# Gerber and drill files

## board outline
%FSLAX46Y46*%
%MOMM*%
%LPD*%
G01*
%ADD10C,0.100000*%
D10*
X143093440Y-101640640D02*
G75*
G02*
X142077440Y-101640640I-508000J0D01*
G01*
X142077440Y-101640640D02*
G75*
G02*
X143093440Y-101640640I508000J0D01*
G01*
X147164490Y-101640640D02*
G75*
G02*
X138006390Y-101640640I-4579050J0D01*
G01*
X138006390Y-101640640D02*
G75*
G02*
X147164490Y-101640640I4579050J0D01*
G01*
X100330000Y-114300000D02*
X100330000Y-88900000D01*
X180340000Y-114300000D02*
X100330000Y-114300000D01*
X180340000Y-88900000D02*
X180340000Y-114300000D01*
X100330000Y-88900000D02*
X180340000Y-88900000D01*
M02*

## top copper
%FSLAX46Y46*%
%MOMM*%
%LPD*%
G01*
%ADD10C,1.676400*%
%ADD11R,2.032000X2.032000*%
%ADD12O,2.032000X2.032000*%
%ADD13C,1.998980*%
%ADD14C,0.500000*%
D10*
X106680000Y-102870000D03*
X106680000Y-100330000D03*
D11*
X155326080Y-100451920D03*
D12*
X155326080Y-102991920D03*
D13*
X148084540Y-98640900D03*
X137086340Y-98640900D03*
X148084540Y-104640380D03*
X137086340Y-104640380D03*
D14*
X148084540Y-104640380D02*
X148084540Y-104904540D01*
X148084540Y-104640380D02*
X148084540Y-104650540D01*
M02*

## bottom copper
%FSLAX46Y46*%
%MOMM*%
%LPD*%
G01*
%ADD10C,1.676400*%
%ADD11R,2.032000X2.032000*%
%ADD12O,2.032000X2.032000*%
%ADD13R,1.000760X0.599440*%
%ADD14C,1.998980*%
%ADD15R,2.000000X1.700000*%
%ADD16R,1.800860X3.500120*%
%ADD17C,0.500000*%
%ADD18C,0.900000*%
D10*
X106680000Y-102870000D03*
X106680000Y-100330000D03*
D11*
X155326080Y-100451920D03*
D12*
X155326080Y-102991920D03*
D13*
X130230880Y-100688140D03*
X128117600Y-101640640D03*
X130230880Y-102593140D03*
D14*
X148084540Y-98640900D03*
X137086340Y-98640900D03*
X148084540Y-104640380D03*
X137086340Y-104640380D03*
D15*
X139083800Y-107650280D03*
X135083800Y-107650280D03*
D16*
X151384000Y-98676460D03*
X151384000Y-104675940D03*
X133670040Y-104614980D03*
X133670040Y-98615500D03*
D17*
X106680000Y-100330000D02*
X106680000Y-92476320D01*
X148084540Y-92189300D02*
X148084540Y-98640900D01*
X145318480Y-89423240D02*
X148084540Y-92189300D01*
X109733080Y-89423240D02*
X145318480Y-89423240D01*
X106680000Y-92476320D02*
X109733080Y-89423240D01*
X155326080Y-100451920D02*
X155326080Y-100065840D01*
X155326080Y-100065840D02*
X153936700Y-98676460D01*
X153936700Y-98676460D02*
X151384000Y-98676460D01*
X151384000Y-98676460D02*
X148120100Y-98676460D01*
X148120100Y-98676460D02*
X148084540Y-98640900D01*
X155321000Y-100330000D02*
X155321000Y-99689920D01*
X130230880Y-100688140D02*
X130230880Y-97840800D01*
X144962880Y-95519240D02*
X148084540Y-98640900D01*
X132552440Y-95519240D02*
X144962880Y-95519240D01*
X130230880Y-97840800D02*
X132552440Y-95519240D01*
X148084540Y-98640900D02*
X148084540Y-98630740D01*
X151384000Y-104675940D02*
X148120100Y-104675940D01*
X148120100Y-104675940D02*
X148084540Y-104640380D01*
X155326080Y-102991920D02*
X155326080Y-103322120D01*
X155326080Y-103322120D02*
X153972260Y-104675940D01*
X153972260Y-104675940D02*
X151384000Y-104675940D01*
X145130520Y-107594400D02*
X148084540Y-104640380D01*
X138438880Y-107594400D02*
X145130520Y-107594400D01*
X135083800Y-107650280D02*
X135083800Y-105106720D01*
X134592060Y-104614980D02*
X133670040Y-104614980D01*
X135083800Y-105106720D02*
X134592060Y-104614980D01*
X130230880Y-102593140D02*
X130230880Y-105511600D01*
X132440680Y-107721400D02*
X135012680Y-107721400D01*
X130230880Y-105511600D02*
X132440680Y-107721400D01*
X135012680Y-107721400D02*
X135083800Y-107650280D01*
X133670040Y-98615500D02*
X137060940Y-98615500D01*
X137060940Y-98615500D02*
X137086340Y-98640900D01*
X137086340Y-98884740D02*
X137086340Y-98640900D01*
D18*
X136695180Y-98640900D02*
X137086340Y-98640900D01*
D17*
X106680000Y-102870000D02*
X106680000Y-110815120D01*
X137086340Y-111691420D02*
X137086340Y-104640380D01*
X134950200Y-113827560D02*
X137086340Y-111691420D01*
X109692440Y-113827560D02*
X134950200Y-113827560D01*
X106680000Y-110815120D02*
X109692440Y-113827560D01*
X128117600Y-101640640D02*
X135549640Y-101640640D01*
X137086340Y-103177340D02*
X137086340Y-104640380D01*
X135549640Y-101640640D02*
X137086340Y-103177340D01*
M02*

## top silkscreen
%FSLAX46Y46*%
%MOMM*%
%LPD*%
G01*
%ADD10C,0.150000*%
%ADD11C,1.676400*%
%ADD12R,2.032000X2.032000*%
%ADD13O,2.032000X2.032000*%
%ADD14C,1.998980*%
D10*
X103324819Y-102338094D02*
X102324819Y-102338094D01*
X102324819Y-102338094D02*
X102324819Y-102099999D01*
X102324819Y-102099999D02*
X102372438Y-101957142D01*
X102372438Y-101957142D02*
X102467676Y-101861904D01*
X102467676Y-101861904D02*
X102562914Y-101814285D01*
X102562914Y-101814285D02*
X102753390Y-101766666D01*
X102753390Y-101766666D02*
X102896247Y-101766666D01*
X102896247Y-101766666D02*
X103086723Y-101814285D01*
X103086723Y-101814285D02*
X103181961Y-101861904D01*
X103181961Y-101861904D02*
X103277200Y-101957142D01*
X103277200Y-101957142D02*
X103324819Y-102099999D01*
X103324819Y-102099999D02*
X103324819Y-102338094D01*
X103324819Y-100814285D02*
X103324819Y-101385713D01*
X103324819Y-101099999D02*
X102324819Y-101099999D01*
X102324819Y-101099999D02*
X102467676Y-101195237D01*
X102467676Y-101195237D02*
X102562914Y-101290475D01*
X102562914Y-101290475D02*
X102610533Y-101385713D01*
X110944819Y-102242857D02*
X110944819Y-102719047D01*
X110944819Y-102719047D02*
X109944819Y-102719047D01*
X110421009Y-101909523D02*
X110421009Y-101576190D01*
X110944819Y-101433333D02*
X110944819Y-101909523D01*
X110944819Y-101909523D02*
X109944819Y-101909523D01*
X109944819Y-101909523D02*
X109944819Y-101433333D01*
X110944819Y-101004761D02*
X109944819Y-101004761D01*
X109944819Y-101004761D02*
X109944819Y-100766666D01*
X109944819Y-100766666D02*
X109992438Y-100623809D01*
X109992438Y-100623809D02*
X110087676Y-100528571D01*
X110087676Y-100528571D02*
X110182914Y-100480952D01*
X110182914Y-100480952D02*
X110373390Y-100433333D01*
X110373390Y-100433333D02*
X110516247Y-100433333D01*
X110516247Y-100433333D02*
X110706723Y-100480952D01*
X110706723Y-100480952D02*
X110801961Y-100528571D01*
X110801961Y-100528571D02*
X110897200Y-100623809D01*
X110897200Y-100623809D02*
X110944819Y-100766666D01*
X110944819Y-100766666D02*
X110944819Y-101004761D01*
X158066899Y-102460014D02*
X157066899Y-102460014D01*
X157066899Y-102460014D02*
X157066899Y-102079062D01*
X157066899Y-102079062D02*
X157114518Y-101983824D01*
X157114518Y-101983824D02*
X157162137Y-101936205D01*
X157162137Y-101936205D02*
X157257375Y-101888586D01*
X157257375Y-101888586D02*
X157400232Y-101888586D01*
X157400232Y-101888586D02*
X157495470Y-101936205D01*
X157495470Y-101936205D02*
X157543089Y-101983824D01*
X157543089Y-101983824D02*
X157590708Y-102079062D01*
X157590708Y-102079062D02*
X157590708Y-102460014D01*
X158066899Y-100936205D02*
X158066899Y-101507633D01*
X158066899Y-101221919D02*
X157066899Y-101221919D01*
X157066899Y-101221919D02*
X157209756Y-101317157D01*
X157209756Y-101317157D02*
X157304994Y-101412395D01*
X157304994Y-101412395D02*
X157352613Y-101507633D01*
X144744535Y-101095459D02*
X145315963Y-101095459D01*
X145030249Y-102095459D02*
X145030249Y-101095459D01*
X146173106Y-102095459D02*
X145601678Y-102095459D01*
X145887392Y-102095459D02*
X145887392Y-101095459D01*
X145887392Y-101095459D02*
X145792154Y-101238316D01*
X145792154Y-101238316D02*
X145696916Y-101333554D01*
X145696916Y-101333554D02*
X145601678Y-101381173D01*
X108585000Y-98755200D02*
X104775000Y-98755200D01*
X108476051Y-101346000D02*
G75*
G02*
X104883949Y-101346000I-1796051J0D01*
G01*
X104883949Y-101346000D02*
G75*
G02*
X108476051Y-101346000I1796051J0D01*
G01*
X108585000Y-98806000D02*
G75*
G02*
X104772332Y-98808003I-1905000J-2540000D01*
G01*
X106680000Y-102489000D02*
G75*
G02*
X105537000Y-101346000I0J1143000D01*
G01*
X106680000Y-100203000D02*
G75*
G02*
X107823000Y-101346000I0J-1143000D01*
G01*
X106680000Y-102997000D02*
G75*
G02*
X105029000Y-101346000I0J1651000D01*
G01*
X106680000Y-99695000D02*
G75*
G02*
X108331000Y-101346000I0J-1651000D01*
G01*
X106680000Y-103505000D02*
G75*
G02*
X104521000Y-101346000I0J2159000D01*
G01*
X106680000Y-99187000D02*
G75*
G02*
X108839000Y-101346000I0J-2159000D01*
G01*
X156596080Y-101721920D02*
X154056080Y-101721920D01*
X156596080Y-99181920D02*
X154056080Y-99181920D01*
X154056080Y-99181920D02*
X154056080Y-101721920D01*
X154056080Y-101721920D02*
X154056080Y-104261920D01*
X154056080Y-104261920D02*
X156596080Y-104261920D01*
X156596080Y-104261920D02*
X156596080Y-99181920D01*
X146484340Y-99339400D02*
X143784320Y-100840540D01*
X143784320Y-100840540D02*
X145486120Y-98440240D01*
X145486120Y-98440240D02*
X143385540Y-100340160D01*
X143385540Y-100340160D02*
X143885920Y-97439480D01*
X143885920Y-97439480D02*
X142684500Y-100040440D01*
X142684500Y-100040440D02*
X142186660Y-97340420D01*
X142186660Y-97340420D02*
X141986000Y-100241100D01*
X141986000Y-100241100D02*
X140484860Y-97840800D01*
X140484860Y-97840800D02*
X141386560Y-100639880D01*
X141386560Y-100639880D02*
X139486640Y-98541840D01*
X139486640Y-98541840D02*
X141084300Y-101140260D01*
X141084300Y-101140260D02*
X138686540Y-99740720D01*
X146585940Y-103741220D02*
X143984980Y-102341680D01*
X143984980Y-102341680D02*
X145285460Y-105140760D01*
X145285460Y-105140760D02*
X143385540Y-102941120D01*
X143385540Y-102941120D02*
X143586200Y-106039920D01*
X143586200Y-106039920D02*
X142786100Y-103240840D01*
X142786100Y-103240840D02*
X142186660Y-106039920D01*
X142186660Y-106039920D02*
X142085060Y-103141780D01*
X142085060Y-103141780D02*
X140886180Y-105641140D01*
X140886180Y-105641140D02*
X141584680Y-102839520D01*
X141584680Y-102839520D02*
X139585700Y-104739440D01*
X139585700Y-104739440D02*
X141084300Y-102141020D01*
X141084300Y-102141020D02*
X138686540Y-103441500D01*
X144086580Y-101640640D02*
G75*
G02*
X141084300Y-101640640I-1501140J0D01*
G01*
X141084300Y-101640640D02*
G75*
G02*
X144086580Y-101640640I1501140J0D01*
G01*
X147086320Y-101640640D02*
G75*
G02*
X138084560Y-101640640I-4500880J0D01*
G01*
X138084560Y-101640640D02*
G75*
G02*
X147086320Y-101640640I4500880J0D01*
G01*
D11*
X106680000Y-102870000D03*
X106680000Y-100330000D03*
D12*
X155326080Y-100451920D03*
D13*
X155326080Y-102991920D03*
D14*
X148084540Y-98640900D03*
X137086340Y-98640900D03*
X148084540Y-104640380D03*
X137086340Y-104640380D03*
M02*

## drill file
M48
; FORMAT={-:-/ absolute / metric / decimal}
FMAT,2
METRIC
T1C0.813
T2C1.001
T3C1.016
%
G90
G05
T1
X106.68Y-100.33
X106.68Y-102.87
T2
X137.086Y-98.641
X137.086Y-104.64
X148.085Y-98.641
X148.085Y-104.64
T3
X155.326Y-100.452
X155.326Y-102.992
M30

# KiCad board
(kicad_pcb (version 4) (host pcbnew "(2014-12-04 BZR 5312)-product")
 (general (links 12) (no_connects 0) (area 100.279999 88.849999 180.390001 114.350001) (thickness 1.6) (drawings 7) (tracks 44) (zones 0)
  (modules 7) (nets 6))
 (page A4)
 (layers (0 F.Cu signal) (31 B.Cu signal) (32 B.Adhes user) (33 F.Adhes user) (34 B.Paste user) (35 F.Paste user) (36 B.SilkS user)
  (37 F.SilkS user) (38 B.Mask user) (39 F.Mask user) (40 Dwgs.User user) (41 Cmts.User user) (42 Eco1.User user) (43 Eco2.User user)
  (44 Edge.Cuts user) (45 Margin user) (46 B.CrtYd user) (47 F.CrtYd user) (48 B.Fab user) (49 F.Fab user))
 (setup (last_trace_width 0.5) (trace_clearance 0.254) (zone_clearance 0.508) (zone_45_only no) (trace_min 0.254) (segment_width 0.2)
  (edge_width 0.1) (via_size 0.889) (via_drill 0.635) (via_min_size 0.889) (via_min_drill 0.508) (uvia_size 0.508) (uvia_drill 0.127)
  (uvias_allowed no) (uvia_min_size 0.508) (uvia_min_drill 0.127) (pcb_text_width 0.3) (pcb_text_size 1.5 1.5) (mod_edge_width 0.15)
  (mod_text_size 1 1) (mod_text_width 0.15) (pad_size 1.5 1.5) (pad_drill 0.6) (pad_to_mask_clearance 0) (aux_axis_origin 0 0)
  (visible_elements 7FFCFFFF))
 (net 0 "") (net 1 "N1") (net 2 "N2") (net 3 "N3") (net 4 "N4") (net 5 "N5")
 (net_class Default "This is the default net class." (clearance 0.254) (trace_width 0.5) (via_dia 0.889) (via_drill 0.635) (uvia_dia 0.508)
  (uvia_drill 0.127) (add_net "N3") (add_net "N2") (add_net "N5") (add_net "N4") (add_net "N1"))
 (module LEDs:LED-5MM (layer F.Cu) (at 106.68 101.6 90)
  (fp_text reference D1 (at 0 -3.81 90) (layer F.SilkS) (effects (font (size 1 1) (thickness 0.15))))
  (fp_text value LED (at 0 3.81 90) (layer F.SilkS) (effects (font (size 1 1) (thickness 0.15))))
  (fp_line (start 2.8448 1.905) (end 2.8448 -1.905) (layer F.SilkS) (width 0.15))
  (fp_circle (center 0.254 0) (end -1.016 1.27) (layer F.SilkS) (width 0.15))
  (fp_arc (start 0.254 0) (end 2.794 1.905) (angle 286.2) (layer F.SilkS) (width 0.15))
  (fp_arc (start 0.254 0) (end -0.889 0) (angle 90) (layer F.SilkS) (width 0.15))
  (fp_arc (start 0.254 0) (end 1.397 0) (angle 90) (layer F.SilkS) (width 0.15))
  (fp_arc (start 0.254 0) (end -1.397 0) (angle 90) (layer F.SilkS) (width 0.15))
  (fp_arc (start 0.254 0) (end 1.905 0) (angle 90) (layer F.SilkS) (width 0.15))
  (fp_arc (start 0.254 0) (end -1.905 0) (angle 90) (layer F.SilkS) (width 0.15))
  (fp_arc (start 0.254 0) (end 2.413 0) (angle 90) (layer F.SilkS) (width 0.15))
  (pad 1 thru_hole circle (at -1.27 0 90) (size 1.6764 1.6764) (drill 0.8128) (layers *.Cu *.Mask F.SilkS) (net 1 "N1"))
  (pad 2 thru_hole circle (at 1.27 0 90) (size 1.6764 1.6764) (drill 0.8128) (layers *.Cu *.Mask F.SilkS) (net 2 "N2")))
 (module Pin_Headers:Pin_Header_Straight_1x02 (layer F.Cu) (at 155.32608 101.72192 270)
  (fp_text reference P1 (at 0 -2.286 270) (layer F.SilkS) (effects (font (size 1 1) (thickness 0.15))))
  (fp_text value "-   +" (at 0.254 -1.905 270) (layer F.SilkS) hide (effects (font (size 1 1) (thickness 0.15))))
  (fp_line (start 0 -1.27) (end 0 1.27) (layer F.SilkS) (width 0.15))
  (fp_line (start -2.54 -1.27) (end -2.54 1.27) (layer F.SilkS) (width 0.15))
  (fp_line (start -2.54 1.27) (end 0 1.27) (layer F.SilkS) (width 0.15))
  (fp_line (start 0 1.27) (end 2.54 1.27) (layer F.SilkS) (width 0.15))
  (fp_line (start 2.54 1.27) (end 2.54 -1.27) (layer F.SilkS) (width 0.15))
  (fp_line (start 2.54 -1.27) (end -2.54 -1.27) (layer F.SilkS) (width 0.15))
  (pad 1 thru_hole rect (at -1.27 0 270) (size 2.032 2.032) (drill 1.016) (layers *.Cu *.Mask F.SilkS) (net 2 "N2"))
  (pad 2 thru_hole oval (at 1.27 0 270) (size 2.032 2.032) (drill 1.016) (layers *.Cu *.Mask F.SilkS) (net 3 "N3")))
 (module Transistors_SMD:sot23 (layer B.Cu) (at 129.17424 101.64064 270)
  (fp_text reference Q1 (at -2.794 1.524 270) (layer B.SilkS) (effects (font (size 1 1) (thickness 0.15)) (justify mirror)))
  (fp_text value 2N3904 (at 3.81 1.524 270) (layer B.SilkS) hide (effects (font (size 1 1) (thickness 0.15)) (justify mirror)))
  (pad 1 smd rect (at -0.9525 -1.05664 270) (size 0.59944 1.00076) (layers B.Cu B.Paste B.Mask) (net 2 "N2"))
  (pad 3 smd rect (at 0 1.05664 270) (size 0.59944 1.00076) (layers B.Cu B.Paste B.Mask) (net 1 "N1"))
  (pad 2 smd rect (at 0.9525 -1.05664 270) (size 0.59944 1.00076) (layers B.Cu B.Paste B.Mask) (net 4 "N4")))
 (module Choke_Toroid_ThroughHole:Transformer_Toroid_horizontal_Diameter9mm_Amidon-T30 (layer F.Cu) (at 142.58544 101.64064 180)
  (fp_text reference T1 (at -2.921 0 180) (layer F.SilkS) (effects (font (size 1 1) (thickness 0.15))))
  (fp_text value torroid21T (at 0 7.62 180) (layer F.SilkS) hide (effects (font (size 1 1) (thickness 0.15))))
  (fp_line (start -3.8989 2.30124) (end -1.19888 0.8001) (layer F.SilkS) (width 0.15))
  (fp_line (start -1.19888 0.8001) (end -2.90068 3.2004) (layer F.SilkS) (width 0.15))
  (fp_line (start -2.90068 3.2004) (end -0.8001 1.30048) (layer F.SilkS) (width 0.15))
  (fp_line (start -0.8001 1.30048) (end -1.30048 4.20116) (layer F.SilkS) (width 0.15))
  (fp_line (start -1.30048 4.20116) (end -0.09906 1.6002) (layer F.SilkS) (width 0.15))
  (fp_line (start -0.09906 1.6002) (end 0.39878 4.30022) (layer F.SilkS) (width 0.15))
  (fp_line (start 0.39878 4.30022) (end 0.59944 1.39954) (layer F.SilkS) (width 0.15))
  (fp_line (start 0.59944 1.39954) (end 2.10058 3.79984) (layer F.SilkS) (width 0.15))
  (fp_line (start 2.10058 3.79984) (end 1.19888 1.00076) (layer F.SilkS) (width 0.15))
  (fp_line (start 1.19888 1.00076) (end 3.0988 3.0988) (layer F.SilkS) (width 0.15))
  (fp_line (start 3.0988 3.0988) (end 1.50114 0.50038) (layer F.SilkS) (width 0.15))
  (fp_line (start 1.50114 0.50038) (end 3.8989 1.89992) (layer F.SilkS) (width 0.15))
  (fp_line (start -4.0005 -2.10058) (end -1.39954 -0.70104) (layer F.SilkS) (width 0.15))
  (fp_line (start -1.39954 -0.70104) (end -2.70002 -3.50012) (layer F.SilkS) (width 0.15))
  (fp_line (start -2.70002 -3.50012) (end -0.8001 -1.30048) (layer F.SilkS) (width 0.15))
  (fp_line (start -0.8001 -1.30048) (end -1.00076 -4.39928) (layer F.SilkS) (width 0.15))
  (fp_line (start -1.00076 -4.39928) (end -0.20066 -1.6002) (layer F.SilkS) (width 0.15))
  (fp_line (start -0.20066 -1.6002) (end 0.39878 -4.39928) (layer F.SilkS) (width 0.15))
  (fp_line (start 0.39878 -4.39928) (end 0.50038 -1.50114) (layer F.SilkS) (width 0.15))
  (fp_line (start 0.50038 -1.50114) (end 1.69926 -4.0005) (layer F.SilkS) (width 0.15))
  (fp_line (start 1.69926 -4.0005) (end 1.00076 -1.19888) (layer F.SilkS) (width 0.15))
  (fp_line (start 1.00076 -1.19888) (end 2.99974 -3.0988) (layer F.SilkS) (width 0.15))
  (fp_line (start 2.99974 -3.0988) (end 1.50114 -0.50038) (layer F.SilkS) (width 0.15))
  (fp_line (start 1.50114 -0.50038) (end 3.8989 -1.80086) (layer F.SilkS) (width 0.15))
  (fp_circle (center 0 0) (end 1.50114 0) (layer F.SilkS) (width 0.15))
  (fp_circle (center 0 0) (end 4.50088 0) (layer F.SilkS) (width 0.15))
  (pad 1 thru_hole circle (at -5.4991 2.99974 180) (size 1.99898 1.99898) (drill 1.00076) (layers *.Cu *.Mask F.SilkS) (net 2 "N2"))
  (pad 2 thru_hole circle (at 5.4991 2.99974 180) (size 1.99898 1.99898) (drill 1.00076) (layers *.Cu *.Mask F.SilkS) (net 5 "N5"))
  (pad 3 thru_hole circle (at -5.4991 -2.99974 180) (size 1.99898 1.99898) (drill 1.00076) (layers *.Cu *.Mask F.SilkS) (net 3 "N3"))
  (pad 4 thru_hole circle (at 5.4991 -2.99974 180) (size 1.99898 1.99898) (drill 1.00076) (layers *.Cu *.Mask F.SilkS) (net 1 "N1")))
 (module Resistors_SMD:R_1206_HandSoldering (layer B.Cu) (at 137.0838 107.65028 180)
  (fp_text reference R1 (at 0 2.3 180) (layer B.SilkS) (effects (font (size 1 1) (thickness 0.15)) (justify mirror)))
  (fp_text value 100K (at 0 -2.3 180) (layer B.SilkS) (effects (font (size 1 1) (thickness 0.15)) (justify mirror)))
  (pad 1 smd rect (at -2 0 180) (size 2 1.7) (layers B.Cu B.Paste B.Mask) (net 3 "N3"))
  (pad 2 smd rect (at 2 0 180) (size 2 1.7) (layers B.Cu B.Paste B.Mask) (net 4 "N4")))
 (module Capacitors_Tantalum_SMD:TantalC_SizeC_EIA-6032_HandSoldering (layer B.Cu) (at 151.384 101.6762 90)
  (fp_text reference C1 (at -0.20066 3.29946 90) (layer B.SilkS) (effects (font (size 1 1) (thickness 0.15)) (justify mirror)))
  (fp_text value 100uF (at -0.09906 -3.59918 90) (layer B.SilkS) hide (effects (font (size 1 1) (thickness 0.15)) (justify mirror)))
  (pad 2 smd rect (at 2.99974 0 90) (size 3.50012 1.80086) (layers B.Cu B.Paste B.Mask) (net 2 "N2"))
  (pad 1 smd rect (at -2.99974 0 90) (size 3.50012 1.80086) (layers B.Cu B.Paste B.Mask) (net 3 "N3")))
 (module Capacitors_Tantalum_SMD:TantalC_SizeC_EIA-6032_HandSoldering (layer B.Cu) (at 133.67004 101.61524 270)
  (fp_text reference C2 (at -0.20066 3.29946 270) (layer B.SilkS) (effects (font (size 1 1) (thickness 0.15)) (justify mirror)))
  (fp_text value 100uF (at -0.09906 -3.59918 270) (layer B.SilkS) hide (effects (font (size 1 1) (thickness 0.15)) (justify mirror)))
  (pad 2 smd rect (at 2.99974 0 270) (size 3.50012 1.80086) (layers B.Cu B.Paste B.Mask) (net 4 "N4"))
  (pad 1 smd rect (at -2.99974 0 270) (size 3.50012 1.80086) (layers B.Cu B.Paste B.Mask) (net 5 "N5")))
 (gr_circle (center 142.58544 101.64064) (end 143.09344 101.64064) (layer Edge.Cuts) (width 0.1))
 (gr_circle (center 142.58544 101.64064) (end 147.15744 101.89464) (layer Edge.Cuts) (width 0.1))
 (gr_line (start 100.33 114.3) (end 100.33 88.9) (angle 90) (layer Edge.Cuts) (width 0.1))
 (gr_line (start 180.34 114.3) (end 100.33 114.3) (angle 90) (layer Edge.Cuts) (width 0.1))
 (gr_line (start 180.34 88.9) (end 180.34 114.3) (angle 90) (layer Edge.Cuts) (width 0.1))
 (gr_line (start 100.33 88.9) (end 180.34 88.9) (angle 90) (layer Edge.Cuts) (width 0.1))
 (segment (start 106.68 100.33) (end 106.68 92.47632) (width 0.5) (layer B.Cu) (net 2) (status 400000))
 (segment (start 148.08454 92.1893) (end 148.08454 98.6409) (width 0.5) (layer B.Cu) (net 2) (status 800000))
 (segment (start 145.31848 89.42324) (end 148.08454 92.1893) (width 0.5) (layer B.Cu) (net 2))
 (segment (start 109.73308 89.42324) (end 145.31848 89.42324) (width 0.5) (layer B.Cu) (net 2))
 (segment (start 106.68 92.47632) (end 109.73308 89.42324) (width 0.5) (layer B.Cu) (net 2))
 (segment (start 155.32608 100.45192) (end 155.32608 100.06584) (width 0.5) (layer B.Cu) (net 2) (status C00000))
 (segment (start 155.32608 100.06584) (end 153.9367 98.67646) (width 0.5) (layer B.Cu) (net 2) (status 400000))
 (segment (start 153.9367 98.67646) (end 151.384 98.67646) (width 0.5) (layer B.Cu) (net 2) (status 800000))
 (segment (start 151.384 98.67646) (end 148.1201 98.67646) (width 0.5) (layer B.Cu) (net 2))
 (segment (start 148.1201 98.67646) (end 148.08454 98.6409) (width 0.5) (layer B.Cu) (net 2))
 (segment (start 155.321 100.33) (end 155.321 99.68992) (width 0.5) (layer B.Cu) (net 2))
 (segment (start 130.23088 100.68814) (end 130.23088 97.8408) (width 0.5) (layer B.Cu) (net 2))
 (segment (start 144.96288 95.51924) (end 148.08454 98.6409) (width 0.5) (layer B.Cu) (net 2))
 (segment (start 132.55244 95.51924) (end 144.96288 95.51924) (width 0.5) (layer B.Cu) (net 2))
 (segment (start 130.23088 97.8408) (end 132.55244 95.51924) (width 0.5) (layer B.Cu) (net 2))
 (segment (start 148.08454 98.6409) (end 148.08454 98.63074) (width 0.5) (layer B.Cu) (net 2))
 (segment (start 151.384 104.67594) (end 148.1201 104.67594) (width 0.5) (layer B.Cu) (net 3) (status C00000))
 (segment (start 148.1201 104.67594) (end 148.08454 104.64038) (width 0.5) (layer B.Cu) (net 3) (status C00000))
 (segment (start 155.32608 102.99192) (end 155.32608 103.32212) (width 0.5) (layer B.Cu) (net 3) (status C00000))
 (segment (start 155.32608 103.32212) (end 153.97226 104.67594) (width 0.5) (layer B.Cu) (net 3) (status 400000))
 (segment (start 153.97226 104.67594) (end 151.384 104.67594) (width 0.5) (layer B.Cu) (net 3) (status 800000))
 (segment (start 148.08454 104.64038) (end 148.08454 104.90454) (width 0.5) (layer F.Cu) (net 3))
 (segment (start 148.08454 104.64038) (end 148.08454 104.65054) (width 0.5) (layer F.Cu) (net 3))
 (segment (start 145.13052 107.5944) (end 148.08454 104.64038) (width 0.5) (layer B.Cu) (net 3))
 (segment (start 138.43888 107.5944) (end 145.13052 107.5944) (width 0.5) (layer B.Cu) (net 3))
 (segment (start 135.0838 107.65028) (end 135.0838 105.10672) (width 0.5) (layer B.Cu) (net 4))
 (segment (start 134.59206 104.61498) (end 133.67004 104.61498) (width 0.5) (layer B.Cu) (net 4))
 (segment (start 135.0838 105.10672) (end 134.59206 104.61498) (width 0.5) (layer B.Cu) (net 4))
 (segment (start 130.23088 102.59314) (end 130.23088 105.5116) (width 0.5) (layer B.Cu) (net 4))
 (segment (start 132.44068 107.7214) (end 135.01268 107.7214) (width 0.5) (layer B.Cu) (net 4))
 (segment (start 130.23088 105.5116) (end 132.44068 107.7214) (width 0.5) (layer B.Cu) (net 4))
 (segment (start 135.01268 107.7214) (end 135.0838 107.65028) (width 0.5) (layer B.Cu) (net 4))
 (segment (start 133.67004 98.6155) (end 137.06094 98.6155) (width 0.5) (layer B.Cu) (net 5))
 (segment (start 137.06094 98.6155) (end 137.08634 98.6409) (width 0.5) (layer B.Cu) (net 5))
 (segment (start 137.08634 98.88474) (end 137.08634 98.6409) (width 0.5) (layer B.Cu) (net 5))
 (segment (start 136.69518 98.6409) (end 137.08634 98.6409) (width 0.9) (layer B.Cu) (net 5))
 (segment (start 106.68 102.87) (end 106.68 110.81512) (width 0.5) (layer B.Cu) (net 1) (status 400000))
 (segment (start 137.08634 111.69142) (end 137.08634 104.64038) (width 0.5) (layer B.Cu) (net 1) (status 800000))
 (segment (start 134.9502 113.82756) (end 137.08634 111.69142) (width 0.5) (layer B.Cu) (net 1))
 (segment (start 109.69244 113.82756) (end 134.9502 113.82756) (width 0.5) (layer B.Cu) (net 1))
 (segment (start 106.68 110.81512) (end 109.69244 113.82756) (width 0.5) (layer B.Cu) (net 1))
 (segment (start 128.1176 101.64064) (end 135.54964 101.64064) (width 0.5) (layer B.Cu) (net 1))
 (segment (start 137.08634 103.17734) (end 137.08634 104.64038) (width 0.5) (layer B.Cu) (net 1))
 (segment (start 135.54964 101.64064) (end 137.08634 103.17734) (width 0.5) (layer B.Cu) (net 1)))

